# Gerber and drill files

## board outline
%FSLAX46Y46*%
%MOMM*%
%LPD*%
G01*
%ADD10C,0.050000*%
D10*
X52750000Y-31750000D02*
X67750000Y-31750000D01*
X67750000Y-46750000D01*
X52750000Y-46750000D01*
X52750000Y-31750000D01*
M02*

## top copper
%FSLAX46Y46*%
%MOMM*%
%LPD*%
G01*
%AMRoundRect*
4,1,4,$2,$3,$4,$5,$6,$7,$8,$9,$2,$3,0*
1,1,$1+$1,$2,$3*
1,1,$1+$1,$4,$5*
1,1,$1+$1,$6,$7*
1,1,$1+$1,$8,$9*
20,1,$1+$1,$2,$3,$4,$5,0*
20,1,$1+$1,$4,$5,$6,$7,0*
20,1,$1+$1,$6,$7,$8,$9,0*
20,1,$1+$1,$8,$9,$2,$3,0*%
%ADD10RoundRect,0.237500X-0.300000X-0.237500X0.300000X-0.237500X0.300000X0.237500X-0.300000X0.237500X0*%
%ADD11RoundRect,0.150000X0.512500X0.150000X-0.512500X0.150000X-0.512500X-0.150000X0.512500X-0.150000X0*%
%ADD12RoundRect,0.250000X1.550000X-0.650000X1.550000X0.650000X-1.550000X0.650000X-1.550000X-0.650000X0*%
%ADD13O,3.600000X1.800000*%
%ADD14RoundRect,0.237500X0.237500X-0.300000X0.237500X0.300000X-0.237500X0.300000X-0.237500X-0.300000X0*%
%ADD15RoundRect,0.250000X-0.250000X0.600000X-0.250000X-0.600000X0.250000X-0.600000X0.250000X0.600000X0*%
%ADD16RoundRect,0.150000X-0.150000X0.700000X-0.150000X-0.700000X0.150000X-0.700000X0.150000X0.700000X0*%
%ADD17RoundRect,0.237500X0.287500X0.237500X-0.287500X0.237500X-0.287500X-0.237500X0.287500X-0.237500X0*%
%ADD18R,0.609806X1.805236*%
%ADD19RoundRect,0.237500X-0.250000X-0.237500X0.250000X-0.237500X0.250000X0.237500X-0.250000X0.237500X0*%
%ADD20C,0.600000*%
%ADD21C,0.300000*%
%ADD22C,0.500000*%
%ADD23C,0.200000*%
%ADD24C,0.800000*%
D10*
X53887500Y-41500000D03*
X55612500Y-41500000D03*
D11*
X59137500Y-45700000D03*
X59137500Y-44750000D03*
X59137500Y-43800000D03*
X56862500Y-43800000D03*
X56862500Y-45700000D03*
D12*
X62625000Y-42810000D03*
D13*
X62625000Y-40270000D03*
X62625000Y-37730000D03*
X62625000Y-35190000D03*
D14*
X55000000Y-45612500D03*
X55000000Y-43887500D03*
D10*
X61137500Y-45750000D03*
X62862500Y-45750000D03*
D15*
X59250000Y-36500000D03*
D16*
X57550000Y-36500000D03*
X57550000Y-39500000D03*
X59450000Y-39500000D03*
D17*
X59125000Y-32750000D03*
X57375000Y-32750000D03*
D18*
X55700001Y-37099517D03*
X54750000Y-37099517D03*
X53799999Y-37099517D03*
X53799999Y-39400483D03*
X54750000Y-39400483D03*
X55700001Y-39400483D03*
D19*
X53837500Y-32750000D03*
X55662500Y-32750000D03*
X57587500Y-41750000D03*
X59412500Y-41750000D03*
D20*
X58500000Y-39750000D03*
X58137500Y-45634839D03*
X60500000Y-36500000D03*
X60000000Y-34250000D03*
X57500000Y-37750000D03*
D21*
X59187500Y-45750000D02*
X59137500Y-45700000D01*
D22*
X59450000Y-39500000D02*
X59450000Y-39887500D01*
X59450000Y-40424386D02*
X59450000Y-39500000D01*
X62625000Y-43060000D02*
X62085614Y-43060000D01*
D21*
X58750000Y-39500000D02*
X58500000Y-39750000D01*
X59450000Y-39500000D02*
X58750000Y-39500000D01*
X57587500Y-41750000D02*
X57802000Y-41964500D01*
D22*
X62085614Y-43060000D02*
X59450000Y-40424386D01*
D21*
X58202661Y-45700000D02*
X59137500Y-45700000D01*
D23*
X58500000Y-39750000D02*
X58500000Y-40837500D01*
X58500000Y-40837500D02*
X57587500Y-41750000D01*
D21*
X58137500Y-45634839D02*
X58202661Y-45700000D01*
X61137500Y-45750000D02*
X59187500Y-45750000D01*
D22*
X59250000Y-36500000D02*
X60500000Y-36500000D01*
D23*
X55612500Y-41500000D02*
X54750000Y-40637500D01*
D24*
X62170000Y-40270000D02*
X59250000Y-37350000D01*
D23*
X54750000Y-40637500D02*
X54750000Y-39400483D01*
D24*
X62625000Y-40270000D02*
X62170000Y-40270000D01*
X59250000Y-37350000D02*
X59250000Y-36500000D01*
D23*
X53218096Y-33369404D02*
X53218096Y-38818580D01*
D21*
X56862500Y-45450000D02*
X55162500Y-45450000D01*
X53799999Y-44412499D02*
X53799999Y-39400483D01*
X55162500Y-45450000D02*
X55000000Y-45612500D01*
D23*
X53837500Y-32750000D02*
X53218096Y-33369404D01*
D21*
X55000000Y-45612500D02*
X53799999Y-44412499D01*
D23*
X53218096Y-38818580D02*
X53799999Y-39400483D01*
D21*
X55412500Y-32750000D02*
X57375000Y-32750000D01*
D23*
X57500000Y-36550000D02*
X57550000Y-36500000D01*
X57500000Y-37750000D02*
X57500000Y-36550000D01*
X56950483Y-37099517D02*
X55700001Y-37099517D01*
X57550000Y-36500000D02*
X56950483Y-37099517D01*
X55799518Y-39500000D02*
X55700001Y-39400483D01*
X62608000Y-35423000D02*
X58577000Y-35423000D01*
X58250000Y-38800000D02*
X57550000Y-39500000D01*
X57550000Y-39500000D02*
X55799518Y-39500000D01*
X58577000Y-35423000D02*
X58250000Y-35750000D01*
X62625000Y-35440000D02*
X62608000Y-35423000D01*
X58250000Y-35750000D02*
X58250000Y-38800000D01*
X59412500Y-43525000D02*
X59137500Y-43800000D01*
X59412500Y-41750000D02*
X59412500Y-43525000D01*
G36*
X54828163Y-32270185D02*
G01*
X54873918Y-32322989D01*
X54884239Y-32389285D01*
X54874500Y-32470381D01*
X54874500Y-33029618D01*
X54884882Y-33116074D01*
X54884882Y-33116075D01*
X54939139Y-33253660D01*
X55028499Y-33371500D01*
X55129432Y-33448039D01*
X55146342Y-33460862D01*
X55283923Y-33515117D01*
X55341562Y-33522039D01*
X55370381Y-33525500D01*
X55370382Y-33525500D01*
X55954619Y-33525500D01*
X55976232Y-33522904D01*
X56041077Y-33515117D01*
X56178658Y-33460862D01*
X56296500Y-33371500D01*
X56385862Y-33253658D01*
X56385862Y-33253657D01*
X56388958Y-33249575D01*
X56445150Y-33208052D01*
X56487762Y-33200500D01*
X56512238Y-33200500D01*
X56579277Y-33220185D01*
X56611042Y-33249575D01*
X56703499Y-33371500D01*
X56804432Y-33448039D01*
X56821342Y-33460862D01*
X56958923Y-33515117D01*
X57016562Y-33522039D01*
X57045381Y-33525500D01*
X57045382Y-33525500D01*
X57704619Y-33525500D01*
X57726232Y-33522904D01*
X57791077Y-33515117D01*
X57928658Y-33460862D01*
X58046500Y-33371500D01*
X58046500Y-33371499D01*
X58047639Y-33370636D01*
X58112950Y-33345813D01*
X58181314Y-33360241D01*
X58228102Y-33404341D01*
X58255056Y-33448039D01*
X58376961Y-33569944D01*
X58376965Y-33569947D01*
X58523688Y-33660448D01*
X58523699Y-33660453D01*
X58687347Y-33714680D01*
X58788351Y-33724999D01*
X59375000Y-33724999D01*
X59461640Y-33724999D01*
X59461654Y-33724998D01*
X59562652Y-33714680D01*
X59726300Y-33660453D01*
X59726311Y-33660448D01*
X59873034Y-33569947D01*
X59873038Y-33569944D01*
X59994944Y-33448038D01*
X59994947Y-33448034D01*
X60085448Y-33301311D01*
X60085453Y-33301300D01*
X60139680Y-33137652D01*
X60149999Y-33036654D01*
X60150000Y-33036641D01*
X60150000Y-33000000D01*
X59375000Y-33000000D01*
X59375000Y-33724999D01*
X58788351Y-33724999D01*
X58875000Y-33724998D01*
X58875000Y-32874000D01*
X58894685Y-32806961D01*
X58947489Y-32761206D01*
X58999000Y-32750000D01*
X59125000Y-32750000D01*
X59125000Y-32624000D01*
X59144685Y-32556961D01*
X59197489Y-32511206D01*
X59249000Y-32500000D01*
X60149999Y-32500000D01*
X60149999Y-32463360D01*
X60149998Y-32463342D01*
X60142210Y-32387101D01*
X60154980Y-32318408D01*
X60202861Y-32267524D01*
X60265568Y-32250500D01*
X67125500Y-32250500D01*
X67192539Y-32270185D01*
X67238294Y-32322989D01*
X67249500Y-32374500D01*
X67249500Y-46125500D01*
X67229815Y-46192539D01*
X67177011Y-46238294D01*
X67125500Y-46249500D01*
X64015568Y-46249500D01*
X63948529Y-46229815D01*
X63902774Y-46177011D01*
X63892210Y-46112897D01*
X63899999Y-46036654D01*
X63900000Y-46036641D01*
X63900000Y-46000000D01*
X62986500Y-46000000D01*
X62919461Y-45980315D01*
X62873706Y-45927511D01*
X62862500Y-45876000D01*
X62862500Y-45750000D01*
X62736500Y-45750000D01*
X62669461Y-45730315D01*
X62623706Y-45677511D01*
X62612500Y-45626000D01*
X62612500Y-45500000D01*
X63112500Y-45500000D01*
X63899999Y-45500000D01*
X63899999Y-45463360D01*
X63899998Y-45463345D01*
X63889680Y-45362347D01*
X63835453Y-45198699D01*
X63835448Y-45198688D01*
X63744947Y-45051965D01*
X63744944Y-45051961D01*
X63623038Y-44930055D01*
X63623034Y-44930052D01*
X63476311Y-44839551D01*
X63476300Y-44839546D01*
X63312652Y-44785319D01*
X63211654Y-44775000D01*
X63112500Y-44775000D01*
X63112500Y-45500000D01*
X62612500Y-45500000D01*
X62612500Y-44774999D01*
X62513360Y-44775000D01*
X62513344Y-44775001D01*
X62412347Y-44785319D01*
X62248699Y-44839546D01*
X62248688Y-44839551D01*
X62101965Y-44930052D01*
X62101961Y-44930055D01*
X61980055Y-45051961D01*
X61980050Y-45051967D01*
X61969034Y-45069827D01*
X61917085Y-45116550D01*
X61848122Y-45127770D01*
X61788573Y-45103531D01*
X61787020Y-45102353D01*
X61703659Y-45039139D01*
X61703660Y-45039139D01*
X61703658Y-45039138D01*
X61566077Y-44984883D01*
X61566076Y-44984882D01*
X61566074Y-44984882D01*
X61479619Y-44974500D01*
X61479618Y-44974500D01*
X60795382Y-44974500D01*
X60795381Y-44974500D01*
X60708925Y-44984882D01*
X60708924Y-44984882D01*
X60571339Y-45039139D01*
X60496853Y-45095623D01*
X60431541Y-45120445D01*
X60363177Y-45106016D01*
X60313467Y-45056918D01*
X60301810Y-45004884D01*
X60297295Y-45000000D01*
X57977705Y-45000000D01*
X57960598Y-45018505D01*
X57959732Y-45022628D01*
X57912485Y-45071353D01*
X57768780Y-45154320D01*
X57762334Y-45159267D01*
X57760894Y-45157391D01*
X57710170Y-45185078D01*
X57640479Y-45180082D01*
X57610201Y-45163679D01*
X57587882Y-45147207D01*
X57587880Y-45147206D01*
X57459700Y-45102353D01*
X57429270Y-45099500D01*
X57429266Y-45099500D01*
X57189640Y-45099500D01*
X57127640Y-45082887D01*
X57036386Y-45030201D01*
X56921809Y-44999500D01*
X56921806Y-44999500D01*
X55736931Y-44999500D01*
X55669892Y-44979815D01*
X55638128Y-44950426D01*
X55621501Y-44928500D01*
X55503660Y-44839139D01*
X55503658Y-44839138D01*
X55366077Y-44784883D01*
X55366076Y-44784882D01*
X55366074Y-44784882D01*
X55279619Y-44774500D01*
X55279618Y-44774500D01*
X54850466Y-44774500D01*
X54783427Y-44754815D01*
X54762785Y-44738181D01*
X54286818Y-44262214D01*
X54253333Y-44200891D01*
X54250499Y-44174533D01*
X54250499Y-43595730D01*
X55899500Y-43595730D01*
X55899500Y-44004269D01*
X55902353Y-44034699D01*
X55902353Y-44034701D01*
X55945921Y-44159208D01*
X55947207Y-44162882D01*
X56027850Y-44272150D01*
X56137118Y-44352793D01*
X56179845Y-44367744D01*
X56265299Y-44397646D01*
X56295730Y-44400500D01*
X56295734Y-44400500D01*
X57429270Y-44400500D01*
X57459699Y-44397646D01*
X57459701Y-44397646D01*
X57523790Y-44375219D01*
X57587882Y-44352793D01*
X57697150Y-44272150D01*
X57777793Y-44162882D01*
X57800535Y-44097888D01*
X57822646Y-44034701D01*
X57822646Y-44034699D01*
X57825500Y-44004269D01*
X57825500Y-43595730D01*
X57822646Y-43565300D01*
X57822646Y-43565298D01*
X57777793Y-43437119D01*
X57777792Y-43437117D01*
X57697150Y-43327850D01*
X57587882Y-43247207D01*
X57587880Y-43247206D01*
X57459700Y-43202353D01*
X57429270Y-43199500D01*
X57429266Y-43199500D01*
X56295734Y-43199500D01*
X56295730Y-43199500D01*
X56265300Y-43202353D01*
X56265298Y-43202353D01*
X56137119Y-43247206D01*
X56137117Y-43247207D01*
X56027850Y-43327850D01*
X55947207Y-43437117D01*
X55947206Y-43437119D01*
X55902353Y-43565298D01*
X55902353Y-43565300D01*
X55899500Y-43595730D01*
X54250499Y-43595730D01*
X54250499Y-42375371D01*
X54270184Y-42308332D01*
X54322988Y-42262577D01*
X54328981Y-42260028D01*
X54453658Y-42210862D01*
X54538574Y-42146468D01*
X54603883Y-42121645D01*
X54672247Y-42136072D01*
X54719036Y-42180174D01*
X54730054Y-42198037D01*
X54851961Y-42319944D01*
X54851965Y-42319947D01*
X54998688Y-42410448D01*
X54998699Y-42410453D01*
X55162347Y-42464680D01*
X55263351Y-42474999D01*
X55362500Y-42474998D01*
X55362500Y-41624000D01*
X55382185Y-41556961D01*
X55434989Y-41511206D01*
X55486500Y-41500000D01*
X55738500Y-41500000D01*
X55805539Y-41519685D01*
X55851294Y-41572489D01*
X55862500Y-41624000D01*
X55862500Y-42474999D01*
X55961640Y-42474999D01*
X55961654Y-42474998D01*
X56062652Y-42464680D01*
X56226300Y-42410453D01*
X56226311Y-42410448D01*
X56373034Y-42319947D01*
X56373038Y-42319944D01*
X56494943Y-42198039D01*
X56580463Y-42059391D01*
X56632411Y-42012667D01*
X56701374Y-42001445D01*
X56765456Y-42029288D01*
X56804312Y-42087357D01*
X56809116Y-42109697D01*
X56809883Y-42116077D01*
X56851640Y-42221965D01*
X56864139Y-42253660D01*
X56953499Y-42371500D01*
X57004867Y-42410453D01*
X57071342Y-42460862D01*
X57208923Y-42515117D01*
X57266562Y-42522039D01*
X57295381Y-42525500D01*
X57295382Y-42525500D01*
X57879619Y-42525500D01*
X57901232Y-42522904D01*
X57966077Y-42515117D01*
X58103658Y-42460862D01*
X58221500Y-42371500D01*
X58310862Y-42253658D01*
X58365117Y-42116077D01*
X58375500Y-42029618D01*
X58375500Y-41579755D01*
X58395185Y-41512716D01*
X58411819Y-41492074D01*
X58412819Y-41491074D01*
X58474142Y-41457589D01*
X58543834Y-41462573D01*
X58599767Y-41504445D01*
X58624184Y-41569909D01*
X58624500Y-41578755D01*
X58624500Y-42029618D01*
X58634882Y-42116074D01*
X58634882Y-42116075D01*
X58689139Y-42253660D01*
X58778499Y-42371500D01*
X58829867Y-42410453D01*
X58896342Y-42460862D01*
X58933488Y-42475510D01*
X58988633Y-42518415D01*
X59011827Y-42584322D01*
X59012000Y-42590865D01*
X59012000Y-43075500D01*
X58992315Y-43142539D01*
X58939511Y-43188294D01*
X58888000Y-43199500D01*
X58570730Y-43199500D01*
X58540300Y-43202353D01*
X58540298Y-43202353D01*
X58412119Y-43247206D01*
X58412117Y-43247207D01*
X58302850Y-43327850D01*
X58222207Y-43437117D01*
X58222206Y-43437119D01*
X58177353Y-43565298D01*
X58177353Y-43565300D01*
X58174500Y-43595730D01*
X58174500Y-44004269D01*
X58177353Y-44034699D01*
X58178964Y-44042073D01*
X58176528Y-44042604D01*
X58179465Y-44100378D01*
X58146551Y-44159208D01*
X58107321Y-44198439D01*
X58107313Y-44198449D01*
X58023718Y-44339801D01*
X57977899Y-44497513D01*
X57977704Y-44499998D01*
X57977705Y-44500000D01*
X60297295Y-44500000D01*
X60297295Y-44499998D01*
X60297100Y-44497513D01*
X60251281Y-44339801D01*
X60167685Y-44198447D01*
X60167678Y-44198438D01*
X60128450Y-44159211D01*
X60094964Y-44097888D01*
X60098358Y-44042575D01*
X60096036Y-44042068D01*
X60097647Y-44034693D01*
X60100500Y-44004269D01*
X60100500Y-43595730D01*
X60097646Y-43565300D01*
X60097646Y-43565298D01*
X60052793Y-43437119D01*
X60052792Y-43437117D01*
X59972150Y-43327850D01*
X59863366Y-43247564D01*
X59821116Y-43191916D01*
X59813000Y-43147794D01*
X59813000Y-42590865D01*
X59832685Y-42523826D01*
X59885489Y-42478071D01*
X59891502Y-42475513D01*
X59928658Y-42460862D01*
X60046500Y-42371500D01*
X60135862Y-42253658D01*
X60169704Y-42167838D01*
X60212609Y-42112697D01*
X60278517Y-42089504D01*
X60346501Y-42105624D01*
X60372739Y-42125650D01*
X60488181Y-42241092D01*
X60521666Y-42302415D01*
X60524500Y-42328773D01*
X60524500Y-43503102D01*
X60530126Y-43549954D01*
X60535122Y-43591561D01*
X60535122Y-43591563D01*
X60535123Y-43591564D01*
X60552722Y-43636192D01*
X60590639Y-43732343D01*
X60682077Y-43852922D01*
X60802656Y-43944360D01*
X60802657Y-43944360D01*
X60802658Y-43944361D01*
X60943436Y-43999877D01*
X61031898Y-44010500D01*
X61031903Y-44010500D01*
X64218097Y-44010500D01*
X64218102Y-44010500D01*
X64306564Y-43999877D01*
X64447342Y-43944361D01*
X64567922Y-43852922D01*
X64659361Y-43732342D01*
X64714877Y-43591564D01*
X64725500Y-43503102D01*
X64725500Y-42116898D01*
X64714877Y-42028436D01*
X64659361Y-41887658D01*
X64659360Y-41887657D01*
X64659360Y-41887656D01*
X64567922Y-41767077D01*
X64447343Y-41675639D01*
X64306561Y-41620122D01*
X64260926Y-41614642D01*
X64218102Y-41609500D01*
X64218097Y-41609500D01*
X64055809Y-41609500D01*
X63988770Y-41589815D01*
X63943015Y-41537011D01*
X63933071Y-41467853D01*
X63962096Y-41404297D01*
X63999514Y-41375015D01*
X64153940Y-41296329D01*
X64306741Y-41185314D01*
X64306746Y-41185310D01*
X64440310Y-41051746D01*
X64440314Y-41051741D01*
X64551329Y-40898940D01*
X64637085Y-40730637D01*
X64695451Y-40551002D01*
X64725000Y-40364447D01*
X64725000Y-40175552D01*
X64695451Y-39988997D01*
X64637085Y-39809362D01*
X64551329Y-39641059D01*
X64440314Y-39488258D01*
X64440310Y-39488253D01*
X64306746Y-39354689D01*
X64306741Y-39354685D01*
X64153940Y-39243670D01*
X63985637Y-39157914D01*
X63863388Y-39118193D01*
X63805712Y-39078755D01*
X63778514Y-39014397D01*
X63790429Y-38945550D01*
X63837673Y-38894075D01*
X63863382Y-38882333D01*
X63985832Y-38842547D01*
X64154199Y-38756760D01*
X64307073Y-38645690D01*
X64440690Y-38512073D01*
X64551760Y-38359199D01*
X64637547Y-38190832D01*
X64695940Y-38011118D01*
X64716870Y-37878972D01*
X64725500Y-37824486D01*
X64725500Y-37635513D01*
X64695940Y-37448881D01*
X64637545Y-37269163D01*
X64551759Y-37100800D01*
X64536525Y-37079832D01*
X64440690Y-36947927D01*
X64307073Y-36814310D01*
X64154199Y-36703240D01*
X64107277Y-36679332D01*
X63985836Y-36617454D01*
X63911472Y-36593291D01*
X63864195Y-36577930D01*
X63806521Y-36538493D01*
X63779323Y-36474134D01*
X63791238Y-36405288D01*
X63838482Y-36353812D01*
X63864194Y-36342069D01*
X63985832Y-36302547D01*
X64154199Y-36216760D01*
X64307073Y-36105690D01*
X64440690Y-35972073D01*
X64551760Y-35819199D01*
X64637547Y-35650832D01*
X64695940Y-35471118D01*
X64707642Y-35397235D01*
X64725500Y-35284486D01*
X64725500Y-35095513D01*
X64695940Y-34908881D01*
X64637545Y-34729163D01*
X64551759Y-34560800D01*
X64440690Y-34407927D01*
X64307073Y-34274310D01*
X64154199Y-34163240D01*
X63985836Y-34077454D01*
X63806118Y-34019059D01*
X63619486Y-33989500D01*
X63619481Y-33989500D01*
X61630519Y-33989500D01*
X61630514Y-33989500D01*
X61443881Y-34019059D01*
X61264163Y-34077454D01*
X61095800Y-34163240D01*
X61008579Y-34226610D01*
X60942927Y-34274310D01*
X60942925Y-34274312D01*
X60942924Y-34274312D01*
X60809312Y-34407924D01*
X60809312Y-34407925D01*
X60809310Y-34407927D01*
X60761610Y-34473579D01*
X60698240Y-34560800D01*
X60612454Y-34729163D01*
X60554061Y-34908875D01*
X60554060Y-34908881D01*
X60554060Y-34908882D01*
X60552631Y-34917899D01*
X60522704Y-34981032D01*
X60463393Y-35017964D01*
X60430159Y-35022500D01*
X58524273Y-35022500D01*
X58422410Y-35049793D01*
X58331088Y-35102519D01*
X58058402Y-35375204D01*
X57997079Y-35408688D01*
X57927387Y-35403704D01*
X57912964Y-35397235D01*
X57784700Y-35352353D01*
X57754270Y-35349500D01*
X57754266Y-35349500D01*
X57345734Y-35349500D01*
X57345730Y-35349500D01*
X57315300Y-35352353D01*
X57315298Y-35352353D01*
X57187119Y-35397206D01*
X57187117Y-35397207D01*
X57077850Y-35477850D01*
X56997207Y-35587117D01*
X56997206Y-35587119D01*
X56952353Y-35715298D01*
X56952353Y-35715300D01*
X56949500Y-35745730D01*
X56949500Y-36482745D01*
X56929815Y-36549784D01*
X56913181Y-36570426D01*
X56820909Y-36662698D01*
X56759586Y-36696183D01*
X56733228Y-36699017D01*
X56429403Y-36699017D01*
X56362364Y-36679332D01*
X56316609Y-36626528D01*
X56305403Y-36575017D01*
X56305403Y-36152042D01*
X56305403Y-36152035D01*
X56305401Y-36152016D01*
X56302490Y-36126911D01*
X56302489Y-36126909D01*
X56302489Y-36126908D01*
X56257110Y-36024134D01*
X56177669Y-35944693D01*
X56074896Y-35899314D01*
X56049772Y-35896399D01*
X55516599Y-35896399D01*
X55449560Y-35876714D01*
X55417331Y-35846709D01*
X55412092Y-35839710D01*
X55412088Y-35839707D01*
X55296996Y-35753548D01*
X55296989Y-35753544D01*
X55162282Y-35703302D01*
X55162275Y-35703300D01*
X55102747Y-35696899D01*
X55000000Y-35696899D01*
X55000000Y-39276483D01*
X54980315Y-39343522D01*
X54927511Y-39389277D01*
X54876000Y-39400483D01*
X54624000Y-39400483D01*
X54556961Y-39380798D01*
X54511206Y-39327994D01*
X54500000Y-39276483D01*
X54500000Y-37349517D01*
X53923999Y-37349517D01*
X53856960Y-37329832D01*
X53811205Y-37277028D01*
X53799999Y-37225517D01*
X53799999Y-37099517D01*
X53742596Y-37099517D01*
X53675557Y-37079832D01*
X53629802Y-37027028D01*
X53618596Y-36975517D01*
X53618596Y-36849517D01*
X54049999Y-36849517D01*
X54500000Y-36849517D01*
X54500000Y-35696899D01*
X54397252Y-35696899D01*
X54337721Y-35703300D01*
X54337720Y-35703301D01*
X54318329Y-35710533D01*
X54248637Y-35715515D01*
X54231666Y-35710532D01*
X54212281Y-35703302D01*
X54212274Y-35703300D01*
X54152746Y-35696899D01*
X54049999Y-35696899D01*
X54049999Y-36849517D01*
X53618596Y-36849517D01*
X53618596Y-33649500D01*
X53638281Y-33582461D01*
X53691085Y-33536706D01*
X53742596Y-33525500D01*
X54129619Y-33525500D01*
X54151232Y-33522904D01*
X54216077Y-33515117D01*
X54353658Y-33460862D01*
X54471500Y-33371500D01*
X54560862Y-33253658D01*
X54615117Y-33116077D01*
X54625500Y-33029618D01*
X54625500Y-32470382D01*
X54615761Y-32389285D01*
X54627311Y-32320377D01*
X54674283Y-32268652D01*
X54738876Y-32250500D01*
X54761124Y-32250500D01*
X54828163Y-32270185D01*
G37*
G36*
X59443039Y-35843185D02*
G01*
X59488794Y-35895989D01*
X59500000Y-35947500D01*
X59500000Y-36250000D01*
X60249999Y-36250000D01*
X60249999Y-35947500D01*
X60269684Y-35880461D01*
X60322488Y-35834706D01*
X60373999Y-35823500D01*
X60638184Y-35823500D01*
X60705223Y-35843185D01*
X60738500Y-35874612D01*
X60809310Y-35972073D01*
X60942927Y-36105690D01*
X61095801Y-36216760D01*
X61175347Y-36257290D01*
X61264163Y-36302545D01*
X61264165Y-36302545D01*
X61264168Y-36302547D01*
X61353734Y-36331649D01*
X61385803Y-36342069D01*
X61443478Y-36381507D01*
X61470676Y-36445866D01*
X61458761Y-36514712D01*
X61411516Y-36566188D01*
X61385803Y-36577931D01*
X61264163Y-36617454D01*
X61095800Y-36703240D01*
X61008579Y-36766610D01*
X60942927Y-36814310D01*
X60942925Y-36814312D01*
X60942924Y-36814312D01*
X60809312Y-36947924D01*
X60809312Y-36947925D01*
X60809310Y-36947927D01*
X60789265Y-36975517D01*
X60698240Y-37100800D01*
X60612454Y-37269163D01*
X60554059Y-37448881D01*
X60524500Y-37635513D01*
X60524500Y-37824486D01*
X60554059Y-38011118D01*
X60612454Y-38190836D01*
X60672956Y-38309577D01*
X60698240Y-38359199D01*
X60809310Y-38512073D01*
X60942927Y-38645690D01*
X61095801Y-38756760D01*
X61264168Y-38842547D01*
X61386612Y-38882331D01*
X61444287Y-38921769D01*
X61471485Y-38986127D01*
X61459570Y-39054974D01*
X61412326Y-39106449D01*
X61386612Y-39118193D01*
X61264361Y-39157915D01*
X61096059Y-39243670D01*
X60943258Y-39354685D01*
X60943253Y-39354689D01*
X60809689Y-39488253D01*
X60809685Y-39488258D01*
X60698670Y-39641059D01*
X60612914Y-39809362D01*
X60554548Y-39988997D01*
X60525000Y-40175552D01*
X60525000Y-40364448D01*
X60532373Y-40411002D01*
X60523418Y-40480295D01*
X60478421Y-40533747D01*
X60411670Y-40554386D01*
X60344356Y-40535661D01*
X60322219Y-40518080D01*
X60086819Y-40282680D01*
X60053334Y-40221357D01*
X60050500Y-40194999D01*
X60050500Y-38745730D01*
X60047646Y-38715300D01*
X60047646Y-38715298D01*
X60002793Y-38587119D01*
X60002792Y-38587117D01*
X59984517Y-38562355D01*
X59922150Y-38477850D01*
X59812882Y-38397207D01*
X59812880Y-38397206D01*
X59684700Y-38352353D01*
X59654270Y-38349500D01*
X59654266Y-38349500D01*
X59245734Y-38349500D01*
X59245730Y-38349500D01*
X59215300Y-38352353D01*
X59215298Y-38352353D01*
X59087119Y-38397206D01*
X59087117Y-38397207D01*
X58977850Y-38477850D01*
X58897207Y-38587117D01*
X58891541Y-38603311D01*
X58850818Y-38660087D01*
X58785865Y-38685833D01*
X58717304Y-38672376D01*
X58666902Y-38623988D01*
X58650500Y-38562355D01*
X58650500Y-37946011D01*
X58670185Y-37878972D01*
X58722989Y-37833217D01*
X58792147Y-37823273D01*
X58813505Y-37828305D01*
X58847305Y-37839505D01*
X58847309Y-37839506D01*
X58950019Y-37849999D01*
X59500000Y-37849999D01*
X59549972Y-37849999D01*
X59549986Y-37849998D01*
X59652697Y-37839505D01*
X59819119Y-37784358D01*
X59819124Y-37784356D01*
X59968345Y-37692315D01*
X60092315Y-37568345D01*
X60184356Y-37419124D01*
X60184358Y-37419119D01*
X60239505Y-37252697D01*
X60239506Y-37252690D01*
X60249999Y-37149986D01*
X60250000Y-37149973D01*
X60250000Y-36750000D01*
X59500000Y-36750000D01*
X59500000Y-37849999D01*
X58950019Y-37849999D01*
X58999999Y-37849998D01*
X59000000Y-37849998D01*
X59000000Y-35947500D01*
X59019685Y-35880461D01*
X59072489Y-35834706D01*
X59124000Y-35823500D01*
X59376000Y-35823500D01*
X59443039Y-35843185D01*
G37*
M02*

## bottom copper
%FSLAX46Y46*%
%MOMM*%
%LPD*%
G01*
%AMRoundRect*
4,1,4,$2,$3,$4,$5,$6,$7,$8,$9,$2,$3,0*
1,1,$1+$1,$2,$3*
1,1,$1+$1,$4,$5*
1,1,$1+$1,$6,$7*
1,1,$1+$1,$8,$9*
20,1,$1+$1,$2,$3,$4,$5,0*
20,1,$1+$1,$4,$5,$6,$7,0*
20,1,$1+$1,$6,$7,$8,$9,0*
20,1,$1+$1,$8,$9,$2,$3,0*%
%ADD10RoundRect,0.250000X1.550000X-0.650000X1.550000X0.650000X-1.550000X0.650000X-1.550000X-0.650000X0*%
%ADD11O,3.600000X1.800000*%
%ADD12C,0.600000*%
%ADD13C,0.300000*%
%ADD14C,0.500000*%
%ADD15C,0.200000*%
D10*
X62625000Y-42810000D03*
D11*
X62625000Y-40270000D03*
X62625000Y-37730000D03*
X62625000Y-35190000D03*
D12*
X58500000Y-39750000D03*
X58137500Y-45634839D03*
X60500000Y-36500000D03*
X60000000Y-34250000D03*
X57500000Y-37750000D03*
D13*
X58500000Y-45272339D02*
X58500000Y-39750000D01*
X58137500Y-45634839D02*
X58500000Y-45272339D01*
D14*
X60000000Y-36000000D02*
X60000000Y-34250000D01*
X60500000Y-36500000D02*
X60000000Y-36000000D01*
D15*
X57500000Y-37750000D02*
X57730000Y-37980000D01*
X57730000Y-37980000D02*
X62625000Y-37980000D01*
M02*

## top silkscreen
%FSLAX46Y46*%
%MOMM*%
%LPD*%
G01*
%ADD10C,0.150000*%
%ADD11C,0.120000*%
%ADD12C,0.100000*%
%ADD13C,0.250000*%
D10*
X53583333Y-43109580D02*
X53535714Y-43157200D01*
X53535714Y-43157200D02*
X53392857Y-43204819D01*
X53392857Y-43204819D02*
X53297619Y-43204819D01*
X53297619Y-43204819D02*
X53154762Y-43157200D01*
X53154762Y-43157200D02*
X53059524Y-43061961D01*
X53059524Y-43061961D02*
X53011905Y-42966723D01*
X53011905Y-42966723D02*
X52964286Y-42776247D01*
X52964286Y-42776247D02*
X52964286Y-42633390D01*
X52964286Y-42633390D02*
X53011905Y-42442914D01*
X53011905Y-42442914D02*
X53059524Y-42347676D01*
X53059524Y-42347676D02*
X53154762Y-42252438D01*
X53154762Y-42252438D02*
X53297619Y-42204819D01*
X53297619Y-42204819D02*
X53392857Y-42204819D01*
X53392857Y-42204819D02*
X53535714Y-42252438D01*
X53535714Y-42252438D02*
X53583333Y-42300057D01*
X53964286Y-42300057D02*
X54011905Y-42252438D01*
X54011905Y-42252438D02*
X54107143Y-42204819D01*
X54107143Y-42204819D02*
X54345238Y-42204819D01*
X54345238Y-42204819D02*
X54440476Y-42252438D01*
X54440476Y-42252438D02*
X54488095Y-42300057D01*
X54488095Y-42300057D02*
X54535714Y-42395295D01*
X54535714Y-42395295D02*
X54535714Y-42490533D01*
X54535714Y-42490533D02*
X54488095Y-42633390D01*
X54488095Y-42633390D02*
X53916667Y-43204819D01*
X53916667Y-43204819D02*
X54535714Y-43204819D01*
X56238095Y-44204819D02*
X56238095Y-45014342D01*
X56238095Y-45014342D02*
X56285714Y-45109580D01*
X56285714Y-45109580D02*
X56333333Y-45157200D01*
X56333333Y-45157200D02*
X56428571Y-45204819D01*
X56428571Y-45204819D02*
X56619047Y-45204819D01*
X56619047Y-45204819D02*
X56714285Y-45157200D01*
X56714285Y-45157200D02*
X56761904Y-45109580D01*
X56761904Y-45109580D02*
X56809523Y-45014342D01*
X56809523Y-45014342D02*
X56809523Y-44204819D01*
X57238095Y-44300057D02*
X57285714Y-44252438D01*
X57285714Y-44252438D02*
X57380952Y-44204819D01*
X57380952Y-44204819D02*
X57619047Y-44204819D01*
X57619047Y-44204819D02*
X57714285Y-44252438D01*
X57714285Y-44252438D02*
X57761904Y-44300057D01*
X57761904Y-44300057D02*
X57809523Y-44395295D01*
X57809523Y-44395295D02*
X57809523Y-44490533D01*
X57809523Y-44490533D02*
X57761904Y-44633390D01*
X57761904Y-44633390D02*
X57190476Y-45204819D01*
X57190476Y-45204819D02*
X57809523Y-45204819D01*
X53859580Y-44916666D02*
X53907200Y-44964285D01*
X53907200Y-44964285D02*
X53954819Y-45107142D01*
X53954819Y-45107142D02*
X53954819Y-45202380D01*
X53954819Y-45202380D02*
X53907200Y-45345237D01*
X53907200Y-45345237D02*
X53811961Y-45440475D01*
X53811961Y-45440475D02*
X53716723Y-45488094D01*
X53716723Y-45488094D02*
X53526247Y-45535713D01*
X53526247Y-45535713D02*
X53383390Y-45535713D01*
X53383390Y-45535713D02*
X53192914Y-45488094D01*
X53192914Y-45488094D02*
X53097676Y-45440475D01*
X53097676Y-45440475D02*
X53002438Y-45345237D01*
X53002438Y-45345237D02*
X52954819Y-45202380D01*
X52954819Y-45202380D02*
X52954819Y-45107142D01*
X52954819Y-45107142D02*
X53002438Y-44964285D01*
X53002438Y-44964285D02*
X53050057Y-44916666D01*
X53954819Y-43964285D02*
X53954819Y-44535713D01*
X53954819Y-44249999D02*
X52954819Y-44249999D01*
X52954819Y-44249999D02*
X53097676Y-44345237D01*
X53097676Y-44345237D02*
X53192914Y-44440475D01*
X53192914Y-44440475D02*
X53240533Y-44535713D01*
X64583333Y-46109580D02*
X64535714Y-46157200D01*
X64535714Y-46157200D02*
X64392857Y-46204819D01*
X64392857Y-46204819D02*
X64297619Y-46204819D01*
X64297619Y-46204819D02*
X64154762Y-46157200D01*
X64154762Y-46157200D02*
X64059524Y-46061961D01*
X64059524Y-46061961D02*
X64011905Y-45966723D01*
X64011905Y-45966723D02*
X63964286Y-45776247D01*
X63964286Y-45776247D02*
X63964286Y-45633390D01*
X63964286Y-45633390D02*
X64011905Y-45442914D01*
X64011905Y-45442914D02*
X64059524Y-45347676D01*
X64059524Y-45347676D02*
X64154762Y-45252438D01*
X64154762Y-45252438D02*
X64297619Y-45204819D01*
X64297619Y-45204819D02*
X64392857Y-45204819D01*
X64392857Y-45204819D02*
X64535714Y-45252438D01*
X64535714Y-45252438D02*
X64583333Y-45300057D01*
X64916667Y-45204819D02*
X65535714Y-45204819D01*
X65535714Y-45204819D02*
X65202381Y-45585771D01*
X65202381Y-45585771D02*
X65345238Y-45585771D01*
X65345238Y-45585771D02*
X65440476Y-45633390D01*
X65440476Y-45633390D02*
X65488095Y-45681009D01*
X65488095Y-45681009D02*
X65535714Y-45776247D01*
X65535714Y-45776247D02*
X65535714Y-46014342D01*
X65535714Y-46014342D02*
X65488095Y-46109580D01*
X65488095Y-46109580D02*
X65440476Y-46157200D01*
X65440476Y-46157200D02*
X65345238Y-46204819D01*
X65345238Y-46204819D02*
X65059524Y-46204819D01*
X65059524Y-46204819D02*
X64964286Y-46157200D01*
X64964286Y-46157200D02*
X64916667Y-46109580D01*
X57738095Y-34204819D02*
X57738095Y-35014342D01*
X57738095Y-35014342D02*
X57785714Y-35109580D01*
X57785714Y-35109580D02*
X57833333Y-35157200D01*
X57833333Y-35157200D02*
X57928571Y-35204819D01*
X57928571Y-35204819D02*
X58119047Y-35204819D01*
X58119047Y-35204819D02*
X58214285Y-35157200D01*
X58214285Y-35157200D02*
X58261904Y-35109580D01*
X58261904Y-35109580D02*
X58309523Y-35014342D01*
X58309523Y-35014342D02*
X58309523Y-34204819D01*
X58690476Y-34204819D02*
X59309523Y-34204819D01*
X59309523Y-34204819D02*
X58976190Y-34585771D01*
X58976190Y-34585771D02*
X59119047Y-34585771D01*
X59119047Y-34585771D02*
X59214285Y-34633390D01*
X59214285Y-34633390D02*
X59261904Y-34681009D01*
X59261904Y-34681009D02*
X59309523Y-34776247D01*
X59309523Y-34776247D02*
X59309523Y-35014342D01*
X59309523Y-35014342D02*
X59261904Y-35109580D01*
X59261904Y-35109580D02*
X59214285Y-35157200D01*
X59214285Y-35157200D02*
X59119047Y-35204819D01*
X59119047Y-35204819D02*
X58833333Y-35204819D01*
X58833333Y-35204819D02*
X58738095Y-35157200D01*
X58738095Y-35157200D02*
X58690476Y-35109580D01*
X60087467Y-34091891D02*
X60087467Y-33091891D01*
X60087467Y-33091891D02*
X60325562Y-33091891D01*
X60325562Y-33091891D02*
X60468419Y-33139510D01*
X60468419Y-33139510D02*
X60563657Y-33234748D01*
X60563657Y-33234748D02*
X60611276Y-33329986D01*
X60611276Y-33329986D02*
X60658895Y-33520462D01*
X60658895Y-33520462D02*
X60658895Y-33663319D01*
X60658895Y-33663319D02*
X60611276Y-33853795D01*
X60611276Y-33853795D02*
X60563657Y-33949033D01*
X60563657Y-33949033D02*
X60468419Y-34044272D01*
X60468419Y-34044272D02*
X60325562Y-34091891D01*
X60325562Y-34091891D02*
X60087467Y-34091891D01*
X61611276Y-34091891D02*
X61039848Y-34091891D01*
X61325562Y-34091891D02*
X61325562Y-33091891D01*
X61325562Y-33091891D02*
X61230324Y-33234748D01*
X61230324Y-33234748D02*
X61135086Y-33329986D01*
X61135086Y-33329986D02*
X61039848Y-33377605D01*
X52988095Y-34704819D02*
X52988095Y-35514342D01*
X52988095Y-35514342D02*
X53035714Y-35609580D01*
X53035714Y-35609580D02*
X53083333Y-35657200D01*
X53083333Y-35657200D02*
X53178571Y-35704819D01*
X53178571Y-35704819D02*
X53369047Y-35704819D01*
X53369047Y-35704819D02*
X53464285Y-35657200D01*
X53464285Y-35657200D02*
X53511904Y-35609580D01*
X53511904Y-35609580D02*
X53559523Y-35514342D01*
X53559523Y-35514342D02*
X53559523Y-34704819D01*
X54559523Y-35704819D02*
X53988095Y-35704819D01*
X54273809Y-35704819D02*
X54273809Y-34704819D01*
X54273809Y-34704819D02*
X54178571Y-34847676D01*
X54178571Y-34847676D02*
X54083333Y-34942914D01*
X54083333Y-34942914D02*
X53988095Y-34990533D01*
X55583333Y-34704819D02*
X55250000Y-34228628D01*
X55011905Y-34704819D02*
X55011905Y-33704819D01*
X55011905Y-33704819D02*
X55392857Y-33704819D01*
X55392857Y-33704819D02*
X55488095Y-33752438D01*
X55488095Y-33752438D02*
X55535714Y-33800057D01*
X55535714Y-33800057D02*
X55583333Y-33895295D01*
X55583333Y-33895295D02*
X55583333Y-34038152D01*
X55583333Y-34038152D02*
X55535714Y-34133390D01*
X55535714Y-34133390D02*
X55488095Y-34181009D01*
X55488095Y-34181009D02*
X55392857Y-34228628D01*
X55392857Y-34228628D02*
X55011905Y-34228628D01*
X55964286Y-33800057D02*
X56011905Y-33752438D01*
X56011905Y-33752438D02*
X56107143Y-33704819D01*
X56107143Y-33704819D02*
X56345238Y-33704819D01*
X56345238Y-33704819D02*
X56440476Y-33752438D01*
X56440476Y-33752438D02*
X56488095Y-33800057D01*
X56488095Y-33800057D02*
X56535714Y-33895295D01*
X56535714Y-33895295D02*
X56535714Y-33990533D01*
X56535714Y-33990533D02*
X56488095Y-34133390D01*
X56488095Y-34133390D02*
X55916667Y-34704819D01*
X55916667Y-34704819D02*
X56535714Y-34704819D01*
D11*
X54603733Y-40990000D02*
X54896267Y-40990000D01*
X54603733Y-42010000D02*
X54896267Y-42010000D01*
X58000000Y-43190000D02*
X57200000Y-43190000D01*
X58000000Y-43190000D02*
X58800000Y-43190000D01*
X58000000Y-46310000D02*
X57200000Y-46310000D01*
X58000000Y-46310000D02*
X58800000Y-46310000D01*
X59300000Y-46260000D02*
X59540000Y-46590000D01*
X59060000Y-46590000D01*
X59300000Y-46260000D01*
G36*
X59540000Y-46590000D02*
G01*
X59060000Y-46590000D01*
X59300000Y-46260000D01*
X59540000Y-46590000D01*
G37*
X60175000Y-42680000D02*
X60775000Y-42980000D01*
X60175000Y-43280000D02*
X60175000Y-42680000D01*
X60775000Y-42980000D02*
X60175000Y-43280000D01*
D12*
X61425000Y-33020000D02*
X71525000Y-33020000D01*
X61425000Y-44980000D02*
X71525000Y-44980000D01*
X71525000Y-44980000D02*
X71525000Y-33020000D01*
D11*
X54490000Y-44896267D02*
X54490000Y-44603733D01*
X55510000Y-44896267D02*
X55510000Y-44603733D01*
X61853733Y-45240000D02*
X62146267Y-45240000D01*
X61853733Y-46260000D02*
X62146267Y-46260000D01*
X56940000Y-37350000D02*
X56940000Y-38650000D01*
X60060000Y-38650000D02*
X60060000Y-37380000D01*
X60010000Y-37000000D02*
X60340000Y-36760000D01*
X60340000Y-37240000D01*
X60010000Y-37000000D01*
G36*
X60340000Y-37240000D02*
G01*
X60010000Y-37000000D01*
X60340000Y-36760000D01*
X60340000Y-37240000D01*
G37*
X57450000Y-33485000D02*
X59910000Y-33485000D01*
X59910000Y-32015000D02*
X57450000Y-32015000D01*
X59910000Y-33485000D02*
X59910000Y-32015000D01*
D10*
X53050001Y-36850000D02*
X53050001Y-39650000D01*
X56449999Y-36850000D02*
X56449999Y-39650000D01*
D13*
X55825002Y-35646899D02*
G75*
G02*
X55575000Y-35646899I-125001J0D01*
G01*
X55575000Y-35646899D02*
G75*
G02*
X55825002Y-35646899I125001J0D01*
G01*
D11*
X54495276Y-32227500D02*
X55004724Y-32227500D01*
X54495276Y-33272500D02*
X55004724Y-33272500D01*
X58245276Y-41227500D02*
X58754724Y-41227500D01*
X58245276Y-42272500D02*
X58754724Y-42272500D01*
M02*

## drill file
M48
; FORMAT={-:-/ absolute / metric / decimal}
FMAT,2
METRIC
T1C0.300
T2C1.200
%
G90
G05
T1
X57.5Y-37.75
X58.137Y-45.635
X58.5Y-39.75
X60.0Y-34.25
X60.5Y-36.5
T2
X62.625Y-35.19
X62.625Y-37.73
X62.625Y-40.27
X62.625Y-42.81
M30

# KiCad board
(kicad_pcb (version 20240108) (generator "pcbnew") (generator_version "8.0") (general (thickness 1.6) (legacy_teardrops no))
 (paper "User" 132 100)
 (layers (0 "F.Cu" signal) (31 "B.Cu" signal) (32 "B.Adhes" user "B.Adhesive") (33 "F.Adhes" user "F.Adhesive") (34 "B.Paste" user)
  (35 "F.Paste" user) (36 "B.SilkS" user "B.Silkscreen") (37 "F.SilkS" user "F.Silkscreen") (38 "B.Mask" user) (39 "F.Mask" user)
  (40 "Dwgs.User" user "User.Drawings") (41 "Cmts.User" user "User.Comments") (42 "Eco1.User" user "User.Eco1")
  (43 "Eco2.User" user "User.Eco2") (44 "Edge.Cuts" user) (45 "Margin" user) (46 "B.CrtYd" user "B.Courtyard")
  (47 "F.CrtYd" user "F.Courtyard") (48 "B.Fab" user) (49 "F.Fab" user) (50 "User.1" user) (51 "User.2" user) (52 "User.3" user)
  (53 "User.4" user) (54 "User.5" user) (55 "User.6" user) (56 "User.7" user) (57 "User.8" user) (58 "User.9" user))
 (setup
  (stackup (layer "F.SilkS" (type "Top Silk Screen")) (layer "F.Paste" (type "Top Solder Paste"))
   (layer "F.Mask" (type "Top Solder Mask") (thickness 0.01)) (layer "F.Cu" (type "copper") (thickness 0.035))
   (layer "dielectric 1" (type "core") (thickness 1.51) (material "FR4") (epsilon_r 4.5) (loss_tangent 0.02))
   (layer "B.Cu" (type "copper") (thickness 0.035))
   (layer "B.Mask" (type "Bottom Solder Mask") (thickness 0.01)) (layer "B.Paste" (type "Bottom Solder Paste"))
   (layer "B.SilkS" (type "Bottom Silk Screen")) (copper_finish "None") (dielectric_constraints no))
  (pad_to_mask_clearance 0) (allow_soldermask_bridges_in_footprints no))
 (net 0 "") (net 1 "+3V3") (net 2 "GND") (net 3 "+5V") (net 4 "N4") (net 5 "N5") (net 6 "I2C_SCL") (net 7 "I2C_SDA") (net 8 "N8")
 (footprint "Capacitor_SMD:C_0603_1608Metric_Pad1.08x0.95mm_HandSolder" (layer "F.Cu") (at 54.75 41.5)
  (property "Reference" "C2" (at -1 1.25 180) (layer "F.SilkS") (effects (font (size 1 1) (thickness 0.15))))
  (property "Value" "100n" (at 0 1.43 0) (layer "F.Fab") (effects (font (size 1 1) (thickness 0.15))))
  (fp_line (start -0.146267 -0.51) (end 0.146267 -0.51) (stroke (width 0.12) (type solid)) (layer "F.SilkS"))
  (fp_line (start -0.146267 0.51) (end 0.146267 0.51) (stroke (width 0.12) (type solid)) (layer "F.SilkS"))
  (pad "1" smd roundrect (at -0.8625 0) (size 1.075 0.95) (layers "F.Cu" "F.Paste" "F.Mask") (roundrect_rratio 0.25) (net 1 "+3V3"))
  (pad "2" smd roundrect (at 0.8625 0) (size 1.075 0.95) (layers "F.Cu" "F.Paste" "F.Mask") (roundrect_rratio 0.25) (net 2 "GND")))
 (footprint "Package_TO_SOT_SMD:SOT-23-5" (layer "F.Cu") (at 58 44.75 180)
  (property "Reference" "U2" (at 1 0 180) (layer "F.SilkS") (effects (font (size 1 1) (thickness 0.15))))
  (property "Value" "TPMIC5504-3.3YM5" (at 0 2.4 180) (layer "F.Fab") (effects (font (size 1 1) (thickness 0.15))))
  (fp_line (start 0 1.56) (end 0.8 1.56) (stroke (width 0.12) (type solid)) (layer "F.SilkS"))
  (fp_line (start 0 1.56) (end -0.8 1.56) (stroke (width 0.12) (type solid)) (layer "F.SilkS"))
  (fp_line (start 0 -1.56) (end 0.8 -1.56) (stroke (width 0.12) (type solid)) (layer "F.SilkS"))
  (fp_line (start 0 -1.56) (end -0.8 -1.56) (stroke (width 0.12) (type solid)) (layer "F.SilkS"))
  (fp_poly
   (pts (xy -1.3 -1.51) (xy -1.54 -1.84) (xy -1.06 -1.84) (xy -1.3 -1.51)) (stroke (width 0.12) (type solid)) (fill solid) (layer "F.SilkS"))
  (pad "1" smd roundrect (at -1.1375 -0.95 180) (size 1.325 0.6) (layers "F.Cu" "F.Paste" "F.Mask") (roundrect_rratio 0.25) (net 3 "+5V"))
  (pad "2" smd roundrect (at -1.1375 0 180) (size 1.325 0.6) (layers "F.Cu" "F.Paste" "F.Mask") (roundrect_rratio 0.25) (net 2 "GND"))
  (pad "3" smd roundrect (at -1.1375 0.95 180) (size 1.325 0.6) (layers "F.Cu" "F.Paste" "F.Mask") (roundrect_rratio 0.25) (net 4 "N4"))
  (pad "4" smd roundrect (at 1.1375 0.95 180) (size 1.325 0.6) (layers "F.Cu" "F.Paste" "F.Mask") (roundrect_rratio 0.25) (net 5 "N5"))
  (pad "5" smd roundrect (at 1.1375 -0.95 180) (size 1.325 0.6) (layers "F.Cu" "F.Paste" "F.Mask") (roundrect_rratio 0.25) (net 1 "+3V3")))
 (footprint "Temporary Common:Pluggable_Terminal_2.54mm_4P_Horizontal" (layer "F.Cu") (at 59.175 38.78 90)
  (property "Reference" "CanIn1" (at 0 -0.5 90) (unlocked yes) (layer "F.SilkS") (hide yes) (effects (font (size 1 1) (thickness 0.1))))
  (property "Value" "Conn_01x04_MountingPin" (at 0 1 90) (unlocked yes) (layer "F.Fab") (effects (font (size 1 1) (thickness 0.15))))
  (fp_line (start -3.9 1) (end -4.2 1.6) (stroke (width 0.12) (type solid)) (layer "F.SilkS"))
  (fp_line (start -4.5 1) (end -3.9 1) (stroke (width 0.12) (type solid)) (layer "F.SilkS"))
  (fp_line (start -4.2 1.6) (end -4.5 1) (stroke (width 0.12) (type solid)) (layer "F.SilkS"))
  (fp_line (start 5.76 2.25) (end 5.76 12.35) (stroke (width 0.1) (type default)) (layer "F.SilkS"))
  (fp_line (start -6.2 2.25) (end -6.2 12.35) (stroke (width 0.1) (type default)) (layer "F.SilkS"))
  (fp_line (start -6.2 12.35) (end 5.76 12.35) (stroke (width 0.1) (type default)) (layer "F.SilkS"))
  (pad "1" thru_hole roundrect (at -4.03 3.45 90) (size 1.8 3.6) (drill 1.2) (layers "*.Cu" "*.Mask") (remove_unused_layers no)
   (roundrect_rratio 0.138889) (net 3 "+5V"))
  (pad "2" thru_hole oval (at -1.49 3.45 90) (size 1.8 3.6) (drill 1.2) (layers "*.Cu" "*.Mask") (remove_unused_layers no) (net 2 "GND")
   (zone_connect 0))
  (pad "3" thru_hole oval (at 1.05 3.45 90) (size 1.8 3.6) (drill 1.2) (layers "*.Cu" "*.Mask") (remove_unused_layers no) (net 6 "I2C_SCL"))
  (pad "4" thru_hole oval (at 3.59 3.45 90) (size 1.8 3.6) (drill 1.2) (layers "*.Cu" "*.Mask") (remove_unused_layers no) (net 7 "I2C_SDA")))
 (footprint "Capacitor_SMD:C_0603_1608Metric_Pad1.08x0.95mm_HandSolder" (layer "F.Cu") (at 55 44.75 90)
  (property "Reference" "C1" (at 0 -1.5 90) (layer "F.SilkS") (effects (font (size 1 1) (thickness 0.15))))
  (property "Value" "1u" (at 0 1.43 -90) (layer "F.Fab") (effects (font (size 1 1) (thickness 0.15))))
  (fp_line (start -0.146267 -0.51) (end 0.146267 -0.51) (stroke (width 0.12) (type solid)) (layer "F.SilkS"))
  (fp_line (start -0.146267 0.51) (end 0.146267 0.51) (stroke (width 0.12) (type solid)) (layer "F.SilkS"))
  (pad "1" smd roundrect (at -0.8625 0 90) (size 1.075 0.95) (layers "F.Cu" "F.Paste" "F.Mask") (roundrect_rratio 0.25) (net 1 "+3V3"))
  (pad "2" smd roundrect (at 0.8625 0 90) (size 1.075 0.95) (layers "F.Cu" "F.Paste" "F.Mask") (roundrect_rratio 0.25) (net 2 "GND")
   (zone_connect 2)))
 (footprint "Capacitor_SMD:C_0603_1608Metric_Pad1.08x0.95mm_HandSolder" (layer "F.Cu") (at 62 45.75)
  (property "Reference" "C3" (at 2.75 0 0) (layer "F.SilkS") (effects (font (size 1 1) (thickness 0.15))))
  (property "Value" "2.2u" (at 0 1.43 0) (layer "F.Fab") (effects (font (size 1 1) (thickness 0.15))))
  (fp_line (start -0.146267 -0.51) (end 0.146267 -0.51) (stroke (width 0.12) (type solid)) (layer "F.SilkS"))
  (fp_line (start -0.146267 0.51) (end 0.146267 0.51) (stroke (width 0.12) (type solid)) (layer "F.SilkS"))
  (pad "1" smd roundrect (at -0.8625 0) (size 1.075 0.95) (layers "F.Cu" "F.Paste" "F.Mask") (roundrect_rratio 0.25) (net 3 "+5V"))
  (pad "2" smd roundrect (at 0.8625 0) (size 1.075 0.95) (layers "F.Cu" "F.Paste" "F.Mask") (roundrect_rratio 0.25) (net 2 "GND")))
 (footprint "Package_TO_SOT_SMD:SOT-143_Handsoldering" (layer "F.Cu") (at 58.5 38 -90)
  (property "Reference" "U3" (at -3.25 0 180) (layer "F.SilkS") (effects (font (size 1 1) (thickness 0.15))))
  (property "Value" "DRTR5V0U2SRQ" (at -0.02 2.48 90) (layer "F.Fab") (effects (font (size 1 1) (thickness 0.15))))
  (fp_line (start -0.65 1.56) (end 0.65 1.56) (stroke (width 0.12) (type solid)) (layer "F.SilkS"))
  (fp_line (start 0.65 -1.56) (end -0.62 -1.56) (stroke (width 0.12) (type solid)) (layer "F.SilkS"))
  (fp_poly
   (pts (xy -1 -1.51) (xy -1.24 -1.84) (xy -0.76 -1.84) (xy -1 -1.51)) (stroke (width 0.12) (type solid)) (fill solid) (layer "F.SilkS"))
  (pad "1" smd roundrect (at -1.5 -0.75 270) (size 1.7 1) (layers "F.Cu" "F.Paste" "F.Mask") (roundrect_rratio 0.25) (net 2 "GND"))
  (pad "2" smd roundrect (at -1.5 0.95 270) (size 1.7 0.6) (layers "F.Cu" "F.Paste" "F.Mask") (roundrect_rratio 0.25) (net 6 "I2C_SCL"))
  (pad "3" smd roundrect (at 1.5 0.95 270) (size 1.7 0.6) (layers "F.Cu" "F.Paste" "F.Mask") (roundrect_rratio 0.25) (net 7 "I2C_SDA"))
  (pad "4" smd roundrect (at 1.5 -0.95 270) (size 1.7 0.6) (layers "F.Cu" "F.Paste" "F.Mask") (roundrect_rratio 0.25) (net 3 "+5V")))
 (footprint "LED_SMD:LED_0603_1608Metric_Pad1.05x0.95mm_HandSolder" (layer "F.Cu") (at 58.25 32.75 180)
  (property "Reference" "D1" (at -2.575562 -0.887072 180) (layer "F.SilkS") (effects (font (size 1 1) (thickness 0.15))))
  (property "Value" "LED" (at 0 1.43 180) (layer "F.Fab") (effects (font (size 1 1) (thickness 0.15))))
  (fp_line (start 0.8 -0.735) (end -1.66 -0.735) (stroke (width 0.12) (type solid)) (layer "F.SilkS"))
  (fp_line (start -1.66 0.735) (end 0.8 0.735) (stroke (width 0.12) (type solid)) (layer "F.SilkS"))
  (fp_line (start -1.66 -0.735) (end -1.66 0.735) (stroke (width 0.12) (type solid)) (layer "F.SilkS"))
  (pad "1" smd roundrect (at -0.875 0 180) (size 1.05 0.95) (layers "F.Cu" "F.Paste" "F.Mask") (roundrect_rratio 0.25) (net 2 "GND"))
  (pad "2" smd roundrect (at 0.875 0 180) (size 1.05 0.95) (layers "F.Cu" "F.Paste" "F.Mask") (roundrect_rratio 0.25) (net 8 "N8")))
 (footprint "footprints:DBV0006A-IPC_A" (layer "F.Cu") (at 54.75 38.25 -90)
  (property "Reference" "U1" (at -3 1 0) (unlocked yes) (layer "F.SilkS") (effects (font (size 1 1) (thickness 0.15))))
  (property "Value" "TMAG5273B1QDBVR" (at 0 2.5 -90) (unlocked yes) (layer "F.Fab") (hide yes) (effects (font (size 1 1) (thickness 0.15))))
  (fp_line (start -1.4 1.699999) (end 1.4 1.699999) (stroke (width 0.15) (type solid)) (layer "F.SilkS"))
  (fp_line (start -1.4 -1.699999) (end 1.4 -1.699999) (stroke (width 0.15) (type solid)) (layer "F.SilkS"))
  (fp_circle (center -2.603101 -0.950001) (end -2.4781 -0.950001) (stroke (width 0.25) (type solid)) (fill none) (layer "F.SilkS"))
  (pad "1" smd rect (at -1.150483 -0.950001 270) (size 1.805236 0.609806) (layers "F.Cu" "F.Paste" "F.Mask") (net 6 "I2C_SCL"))
  (pad "2" smd rect (at -1.150483 0 270) (size 1.805236 0.609806) (layers "F.Cu" "F.Paste" "F.Mask") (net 2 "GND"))
  (pad "3" smd rect (at -1.150483 0.950001 270) (size 1.805236 0.609806) (layers "F.Cu" "F.Paste" "F.Mask") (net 2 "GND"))
  (pad "4" smd rect (at 1.150483 0.950001 270) (size 1.805236 0.609806) (layers "F.Cu" "F.Paste" "F.Mask") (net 1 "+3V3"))
  (pad "5" smd rect (at 1.150483 0 270) (size 1.805236 0.609806) (layers "F.Cu" "F.Paste" "F.Mask") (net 2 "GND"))
  (pad "6" smd rect (at 1.150483 -0.950001 270) (size 1.805236 0.609806) (layers "F.Cu" "F.Paste" "F.Mask") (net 7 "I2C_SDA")))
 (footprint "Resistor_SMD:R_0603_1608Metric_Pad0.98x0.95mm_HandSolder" (layer "F.Cu") (at 54.75 32.75)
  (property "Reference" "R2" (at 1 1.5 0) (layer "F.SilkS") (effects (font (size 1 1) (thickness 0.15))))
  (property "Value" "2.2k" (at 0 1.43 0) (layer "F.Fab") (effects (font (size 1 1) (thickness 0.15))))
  (fp_line (start -0.254724 -0.5225) (end 0.254724 -0.5225) (stroke (width 0.12) (type solid)) (layer "F.SilkS"))
  (fp_line (start -0.254724 0.5225) (end 0.254724 0.5225) (stroke (width 0.12) (type solid)) (layer "F.SilkS"))
  (pad "1" smd roundrect (at -0.9125 0) (size 0.975 0.95) (layers "F.Cu" "F.Paste" "F.Mask") (roundrect_rratio 0.25) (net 1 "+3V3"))
  (pad "2" smd roundrect (at 0.9125 0) (size 0.975 0.95) (layers "F.Cu" "F.Paste" "F.Mask") (roundrect_rratio 0.25) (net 8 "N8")))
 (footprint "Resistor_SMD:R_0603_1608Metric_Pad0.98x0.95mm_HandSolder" (layer "F.Cu") (at 58.5 41.75)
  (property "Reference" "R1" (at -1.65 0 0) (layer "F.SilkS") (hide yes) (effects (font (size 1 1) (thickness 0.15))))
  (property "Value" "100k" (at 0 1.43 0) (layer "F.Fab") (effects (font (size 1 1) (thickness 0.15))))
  (fp_line (start -0.254724 -0.5225) (end 0.254724 -0.5225) (stroke (width 0.12) (type solid)) (layer "F.SilkS"))
  (fp_line (start -0.254724 0.5225) (end 0.254724 0.5225) (stroke (width 0.12) (type solid)) (layer "F.SilkS"))
  (pad "1" smd roundrect (at -0.9125 0) (size 0.975 0.95) (layers "F.Cu" "F.Paste" "F.Mask") (roundrect_rratio 0.25) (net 3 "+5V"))
  (pad "2" smd roundrect (at 0.9125 0) (size 0.975 0.95) (layers "F.Cu" "F.Paste" "F.Mask") (roundrect_rratio 0.25) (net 4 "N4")))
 (gr_rect (start 52.75 31.75) (end 67.75 46.75) (stroke (width 0.05) (type default)) (fill none) (layer "Edge.Cuts"))
 (segment (start 59.1875 45.75) (end 59.1375 45.7) (width 0.3) (layer "F.Cu") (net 3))
 (segment (start 59.45 39.5) (end 59.45 39.8875) (width 0.5) (layer "F.Cu") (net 3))
 (segment (start 59.45 40.424386) (end 59.45 39.5) (width 0.5) (layer "F.Cu") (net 3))
 (segment (start 62.625 43.06) (end 62.085614 43.06) (width 0.5) (layer "F.Cu") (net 3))
 (segment (start 58.75 39.5) (end 58.5 39.75) (width 0.3) (layer "F.Cu") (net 3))
 (segment (start 59.45 39.5) (end 58.75 39.5) (width 0.3) (layer "F.Cu") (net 3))
 (segment (start 57.5875 41.75) (end 57.802 41.9645) (width 0.3) (layer "F.Cu") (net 3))
 (segment (start 62.085614 43.06) (end 59.45 40.424386) (width 0.5) (layer "F.Cu") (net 3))
 (segment (start 58.202661 45.7) (end 59.1375 45.7) (width 0.3) (layer "F.Cu") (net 3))
 (segment (start 58.5 39.75) (end 58.5 40.8375) (width 0.2) (layer "F.Cu") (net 3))
 (segment (start 58.5 40.8375) (end 57.5875 41.75) (width 0.2) (layer "F.Cu") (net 3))
 (segment (start 58.1375 45.634839) (end 58.202661 45.7) (width 0.3) (layer "F.Cu") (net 3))
 (segment (start 61.1375 45.75) (end 59.1875 45.75) (width 0.3) (layer "F.Cu") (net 3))
 (via (at 58.5 39.75) (size 0.6) (drill 0.3) (layers "F.Cu" "B.Cu") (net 3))
 (via (at 58.1375 45.634839) (size 0.6) (drill 0.3) (layers "F.Cu" "B.Cu") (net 3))
 (segment (start 58.5 45.272339) (end 58.5 39.75) (width 0.3) (layer "B.Cu") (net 3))
 (segment (start 58.1375 45.634839) (end 58.5 45.272339) (width 0.3) (layer "B.Cu") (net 3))
 (segment (start 59.25 36.5) (end 60.5 36.5) (width 0.5) (layer "F.Cu") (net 2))
 (segment (start 55.6125 41.5) (end 54.75 40.6375) (width 0.2) (layer "F.Cu") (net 2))
 (segment (start 62.17 40.27) (end 59.25 37.35) (width 0.8) (layer "F.Cu") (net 2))
 (segment (start 54.75 40.6375) (end 54.75 39.400483) (width 0.2) (layer "F.Cu") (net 2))
 (segment (start 62.625 40.27) (end 62.17 40.27) (width 0.8) (layer "F.Cu") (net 2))
 (segment (start 59.25 37.35) (end 59.25 36.5) (width 0.8) (layer "F.Cu") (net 2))
 (via (at 60.5 36.5) (size 0.6) (drill 0.3) (layers "F.Cu" "B.Cu") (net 2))
 (via (at 60 34.25) (size 0.6) (drill 0.3) (layers "F.Cu" "B.Cu") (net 2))
 (segment (start 60 36) (end 60 34.25) (width 0.5) (layer "B.Cu") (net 2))
 (segment (start 60.5 36.5) (end 60 36) (width 0.5) (layer "B.Cu") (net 2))
 (segment (start 53.218096 33.369404) (end 53.218096 38.81858) (width 0.2) (layer "F.Cu") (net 1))
 (segment (start 56.8625 45.45) (end 55.1625 45.45) (width 0.3) (layer "F.Cu") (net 1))
 (segment (start 53.799999 44.412499) (end 53.799999 39.400483) (width 0.3) (layer "F.Cu") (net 1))
 (segment (start 55.1625 45.45) (end 55 45.6125) (width 0.3) (layer "F.Cu") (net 1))
 (segment (start 53.8375 32.75) (end 53.218096 33.369404) (width 0.2) (layer "F.Cu") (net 1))
 (segment (start 55 45.6125) (end 53.799999 44.412499) (width 0.3) (layer "F.Cu") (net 1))
 (segment (start 53.218096 38.81858) (end 53.799999 39.400483) (width 0.2) (layer "F.Cu") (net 1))
 (segment (start 55.4125 32.75) (end 57.375 32.75) (width 0.3) (layer "F.Cu") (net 8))
 (segment (start 57.5 36.55) (end 57.55 36.5) (width 0.2) (layer "F.Cu") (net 6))
 (segment (start 57.5 37.75) (end 57.5 36.55) (width 0.2) (layer "F.Cu") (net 6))
 (segment (start 56.950483 37.099517) (end 55.700001 37.099517) (width 0.2) (layer "F.Cu") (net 6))
 (segment (start 57.55 36.5) (end 56.950483 37.099517) (width 0.2) (layer "F.Cu") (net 6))
 (via (at 57.5 37.75) (size 0.6) (drill 0.3) (layers "F.Cu" "B.Cu") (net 6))
 (segment (start 57.5 37.75) (end 57.73 37.98) (width 0.2) (layer "B.Cu") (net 6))
 (segment (start 57.73 37.98) (end 62.625 37.98) (width 0.2) (layer "B.Cu") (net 6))
 (segment (start 55.799518 39.5) (end 55.700001 39.400483) (width 0.2) (layer "F.Cu") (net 7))
 (segment (start 62.608 35.423) (end 58.577 35.423) (width 0.2) (layer "F.Cu") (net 7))
 (segment (start 58.25 38.8) (end 57.55 39.5) (width 0.2) (layer "F.Cu") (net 7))
 (segment (start 57.55 39.5) (end 55.799518 39.5) (width 0.2) (layer "F.Cu") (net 7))
 (segment (start 58.577 35.423) (end 58.25 35.75) (width 0.2) (layer "F.Cu") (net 7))
 (segment (start 62.625 35.44) (end 62.608 35.423) (width 0.2) (layer "F.Cu") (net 7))
 (segment (start 58.25 35.75) (end 58.25 38.8) (width 0.2) (layer "F.Cu") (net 7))
 (segment (start 59.4125 43.525) (end 59.1375 43.8) (width 0.2) (layer "F.Cu") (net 4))
 (segment (start 59.4125 41.75) (end 59.4125 43.525) (width 0.2) (layer "F.Cu") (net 4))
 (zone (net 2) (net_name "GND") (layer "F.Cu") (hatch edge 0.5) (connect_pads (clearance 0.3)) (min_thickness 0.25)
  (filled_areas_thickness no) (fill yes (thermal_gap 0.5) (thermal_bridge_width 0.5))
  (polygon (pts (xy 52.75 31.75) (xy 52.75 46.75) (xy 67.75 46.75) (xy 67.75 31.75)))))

